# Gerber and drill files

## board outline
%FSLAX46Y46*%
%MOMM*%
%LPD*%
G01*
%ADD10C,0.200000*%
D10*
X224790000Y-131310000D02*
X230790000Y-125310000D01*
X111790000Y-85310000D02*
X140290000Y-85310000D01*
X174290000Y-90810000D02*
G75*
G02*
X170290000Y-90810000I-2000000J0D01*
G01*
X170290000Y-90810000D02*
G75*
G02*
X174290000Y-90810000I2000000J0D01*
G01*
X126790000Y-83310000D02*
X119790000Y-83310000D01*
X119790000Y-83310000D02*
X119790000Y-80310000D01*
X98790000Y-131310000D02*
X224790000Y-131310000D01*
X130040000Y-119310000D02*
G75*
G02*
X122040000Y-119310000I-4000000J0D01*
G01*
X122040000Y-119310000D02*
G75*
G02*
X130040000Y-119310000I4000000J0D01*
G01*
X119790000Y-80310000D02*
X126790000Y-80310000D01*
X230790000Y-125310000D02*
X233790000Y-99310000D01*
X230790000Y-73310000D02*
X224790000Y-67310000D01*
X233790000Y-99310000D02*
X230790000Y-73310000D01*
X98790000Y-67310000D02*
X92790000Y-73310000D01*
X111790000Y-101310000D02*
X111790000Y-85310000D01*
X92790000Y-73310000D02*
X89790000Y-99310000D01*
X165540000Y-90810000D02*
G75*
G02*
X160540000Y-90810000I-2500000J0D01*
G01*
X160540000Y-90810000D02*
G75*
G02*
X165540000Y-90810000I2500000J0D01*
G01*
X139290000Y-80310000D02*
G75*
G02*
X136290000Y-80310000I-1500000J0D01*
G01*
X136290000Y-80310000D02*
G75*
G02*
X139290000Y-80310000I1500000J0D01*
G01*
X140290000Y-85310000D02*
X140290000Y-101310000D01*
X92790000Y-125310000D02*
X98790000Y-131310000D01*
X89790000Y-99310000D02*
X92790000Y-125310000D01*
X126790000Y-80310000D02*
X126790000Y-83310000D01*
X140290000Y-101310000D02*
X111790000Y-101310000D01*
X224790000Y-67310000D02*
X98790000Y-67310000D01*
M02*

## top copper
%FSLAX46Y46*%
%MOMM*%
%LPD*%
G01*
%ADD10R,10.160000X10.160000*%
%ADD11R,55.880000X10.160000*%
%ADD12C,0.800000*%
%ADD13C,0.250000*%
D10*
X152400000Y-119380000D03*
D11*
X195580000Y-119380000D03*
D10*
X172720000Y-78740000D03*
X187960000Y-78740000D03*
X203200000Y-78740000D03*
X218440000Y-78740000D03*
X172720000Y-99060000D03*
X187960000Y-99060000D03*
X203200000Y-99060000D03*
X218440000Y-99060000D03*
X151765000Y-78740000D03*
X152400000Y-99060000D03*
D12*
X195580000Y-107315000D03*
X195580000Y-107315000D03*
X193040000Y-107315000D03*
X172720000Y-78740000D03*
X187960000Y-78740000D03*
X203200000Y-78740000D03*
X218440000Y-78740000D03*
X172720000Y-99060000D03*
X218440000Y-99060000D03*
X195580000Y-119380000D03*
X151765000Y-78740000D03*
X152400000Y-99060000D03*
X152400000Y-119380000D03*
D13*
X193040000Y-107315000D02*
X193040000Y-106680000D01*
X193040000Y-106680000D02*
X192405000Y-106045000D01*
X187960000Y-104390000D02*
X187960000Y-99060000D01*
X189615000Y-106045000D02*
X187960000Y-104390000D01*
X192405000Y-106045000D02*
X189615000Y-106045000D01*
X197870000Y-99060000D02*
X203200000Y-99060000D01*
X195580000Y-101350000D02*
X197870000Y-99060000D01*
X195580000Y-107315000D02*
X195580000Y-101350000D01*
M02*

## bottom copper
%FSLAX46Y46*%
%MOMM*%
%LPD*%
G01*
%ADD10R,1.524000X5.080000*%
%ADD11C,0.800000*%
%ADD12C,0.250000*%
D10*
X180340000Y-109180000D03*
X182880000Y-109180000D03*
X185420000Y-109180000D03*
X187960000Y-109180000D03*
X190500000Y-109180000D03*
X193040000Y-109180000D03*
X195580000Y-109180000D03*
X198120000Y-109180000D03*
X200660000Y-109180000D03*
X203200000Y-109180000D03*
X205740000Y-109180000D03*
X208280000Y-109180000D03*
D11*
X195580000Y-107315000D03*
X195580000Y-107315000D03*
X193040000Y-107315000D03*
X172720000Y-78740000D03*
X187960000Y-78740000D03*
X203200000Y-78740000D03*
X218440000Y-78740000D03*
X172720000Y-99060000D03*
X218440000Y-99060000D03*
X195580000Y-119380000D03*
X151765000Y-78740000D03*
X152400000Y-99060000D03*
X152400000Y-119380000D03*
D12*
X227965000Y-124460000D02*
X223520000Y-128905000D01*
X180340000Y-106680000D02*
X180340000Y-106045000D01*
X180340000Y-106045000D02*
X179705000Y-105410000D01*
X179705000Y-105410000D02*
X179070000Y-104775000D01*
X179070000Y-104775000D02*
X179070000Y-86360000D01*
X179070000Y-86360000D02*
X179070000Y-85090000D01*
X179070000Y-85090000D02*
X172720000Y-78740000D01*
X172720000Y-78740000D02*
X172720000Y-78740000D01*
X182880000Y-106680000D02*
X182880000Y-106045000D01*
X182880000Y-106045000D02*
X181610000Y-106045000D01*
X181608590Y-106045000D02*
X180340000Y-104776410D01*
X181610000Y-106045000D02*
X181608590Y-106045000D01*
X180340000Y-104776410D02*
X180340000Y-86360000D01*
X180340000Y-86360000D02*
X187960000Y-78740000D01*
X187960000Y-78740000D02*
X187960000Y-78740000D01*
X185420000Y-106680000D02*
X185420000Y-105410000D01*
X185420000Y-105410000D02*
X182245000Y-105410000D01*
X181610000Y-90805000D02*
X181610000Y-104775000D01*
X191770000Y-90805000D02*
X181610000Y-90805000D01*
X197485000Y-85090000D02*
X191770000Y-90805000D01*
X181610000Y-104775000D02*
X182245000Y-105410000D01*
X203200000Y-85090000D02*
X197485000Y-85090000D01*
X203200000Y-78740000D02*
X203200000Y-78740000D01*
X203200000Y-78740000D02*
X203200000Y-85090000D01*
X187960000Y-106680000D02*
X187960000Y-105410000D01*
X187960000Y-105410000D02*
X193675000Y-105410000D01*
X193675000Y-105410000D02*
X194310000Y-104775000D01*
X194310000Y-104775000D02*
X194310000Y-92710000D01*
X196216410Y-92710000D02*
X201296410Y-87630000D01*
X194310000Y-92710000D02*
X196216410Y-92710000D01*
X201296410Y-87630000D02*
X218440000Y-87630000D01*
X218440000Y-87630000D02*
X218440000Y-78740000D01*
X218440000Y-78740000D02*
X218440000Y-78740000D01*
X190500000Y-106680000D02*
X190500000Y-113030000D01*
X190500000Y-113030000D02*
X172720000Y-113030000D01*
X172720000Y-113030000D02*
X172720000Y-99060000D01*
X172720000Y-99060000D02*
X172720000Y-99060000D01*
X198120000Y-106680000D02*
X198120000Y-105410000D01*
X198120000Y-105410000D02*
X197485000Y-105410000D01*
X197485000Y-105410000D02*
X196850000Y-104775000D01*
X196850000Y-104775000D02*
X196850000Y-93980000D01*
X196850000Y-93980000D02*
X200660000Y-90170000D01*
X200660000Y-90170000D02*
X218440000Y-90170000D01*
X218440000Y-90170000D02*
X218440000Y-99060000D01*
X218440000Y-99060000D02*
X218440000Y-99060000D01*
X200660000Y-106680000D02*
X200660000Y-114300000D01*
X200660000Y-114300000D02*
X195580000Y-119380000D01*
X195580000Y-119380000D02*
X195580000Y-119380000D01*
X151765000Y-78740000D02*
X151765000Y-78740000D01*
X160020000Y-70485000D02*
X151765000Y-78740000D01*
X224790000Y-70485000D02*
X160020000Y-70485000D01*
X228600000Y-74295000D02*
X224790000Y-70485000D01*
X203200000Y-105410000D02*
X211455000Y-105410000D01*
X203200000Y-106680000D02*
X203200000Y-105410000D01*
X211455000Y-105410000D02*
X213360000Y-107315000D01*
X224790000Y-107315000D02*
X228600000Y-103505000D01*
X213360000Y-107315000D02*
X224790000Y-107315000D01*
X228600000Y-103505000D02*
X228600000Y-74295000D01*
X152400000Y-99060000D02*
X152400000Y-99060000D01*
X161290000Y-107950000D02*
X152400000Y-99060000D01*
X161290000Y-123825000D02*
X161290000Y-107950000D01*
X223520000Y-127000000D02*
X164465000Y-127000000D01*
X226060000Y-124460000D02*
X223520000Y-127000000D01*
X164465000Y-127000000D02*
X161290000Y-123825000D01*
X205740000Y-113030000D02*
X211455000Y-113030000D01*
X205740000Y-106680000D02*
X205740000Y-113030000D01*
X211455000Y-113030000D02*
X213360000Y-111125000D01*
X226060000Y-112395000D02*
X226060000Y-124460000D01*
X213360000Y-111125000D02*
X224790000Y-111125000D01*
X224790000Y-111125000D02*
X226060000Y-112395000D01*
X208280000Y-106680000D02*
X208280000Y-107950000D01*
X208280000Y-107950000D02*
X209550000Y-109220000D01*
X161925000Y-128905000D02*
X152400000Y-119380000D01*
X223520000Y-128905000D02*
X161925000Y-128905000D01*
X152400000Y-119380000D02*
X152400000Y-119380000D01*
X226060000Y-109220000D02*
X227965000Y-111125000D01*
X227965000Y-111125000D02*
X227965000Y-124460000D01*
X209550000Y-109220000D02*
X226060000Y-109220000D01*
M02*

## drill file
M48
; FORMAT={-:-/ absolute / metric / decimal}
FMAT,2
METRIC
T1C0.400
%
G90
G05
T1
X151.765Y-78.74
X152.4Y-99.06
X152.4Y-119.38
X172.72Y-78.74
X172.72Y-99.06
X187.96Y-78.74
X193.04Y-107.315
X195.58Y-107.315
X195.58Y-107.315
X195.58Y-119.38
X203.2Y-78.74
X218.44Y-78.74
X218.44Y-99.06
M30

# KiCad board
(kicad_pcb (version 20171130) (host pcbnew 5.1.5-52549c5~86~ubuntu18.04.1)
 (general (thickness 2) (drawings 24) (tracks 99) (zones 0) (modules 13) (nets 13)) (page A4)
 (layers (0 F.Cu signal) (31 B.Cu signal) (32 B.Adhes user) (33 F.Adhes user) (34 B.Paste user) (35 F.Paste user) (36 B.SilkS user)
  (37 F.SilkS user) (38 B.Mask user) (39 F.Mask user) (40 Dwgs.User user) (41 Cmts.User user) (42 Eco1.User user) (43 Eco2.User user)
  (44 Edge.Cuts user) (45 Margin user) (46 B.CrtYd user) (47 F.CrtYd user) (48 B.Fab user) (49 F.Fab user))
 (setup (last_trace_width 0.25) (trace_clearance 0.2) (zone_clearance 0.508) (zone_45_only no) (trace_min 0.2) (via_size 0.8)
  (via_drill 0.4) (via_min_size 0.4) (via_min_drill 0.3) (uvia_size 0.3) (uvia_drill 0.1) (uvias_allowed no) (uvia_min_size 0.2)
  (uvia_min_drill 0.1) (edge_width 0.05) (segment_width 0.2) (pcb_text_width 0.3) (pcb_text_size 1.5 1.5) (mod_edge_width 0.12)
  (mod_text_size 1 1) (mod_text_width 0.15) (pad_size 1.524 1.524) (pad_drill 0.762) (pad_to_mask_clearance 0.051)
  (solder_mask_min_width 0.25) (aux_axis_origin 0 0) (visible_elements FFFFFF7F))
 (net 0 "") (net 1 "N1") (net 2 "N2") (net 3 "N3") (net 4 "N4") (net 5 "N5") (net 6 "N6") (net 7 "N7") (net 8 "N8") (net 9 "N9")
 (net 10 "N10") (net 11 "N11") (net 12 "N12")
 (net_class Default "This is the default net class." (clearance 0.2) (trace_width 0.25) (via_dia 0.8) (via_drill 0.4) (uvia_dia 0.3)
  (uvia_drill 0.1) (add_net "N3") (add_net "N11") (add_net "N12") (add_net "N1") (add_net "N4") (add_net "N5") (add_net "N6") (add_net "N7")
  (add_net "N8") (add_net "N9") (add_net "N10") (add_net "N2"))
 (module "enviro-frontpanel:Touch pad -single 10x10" (layer F.Cu) (at 152.4 127)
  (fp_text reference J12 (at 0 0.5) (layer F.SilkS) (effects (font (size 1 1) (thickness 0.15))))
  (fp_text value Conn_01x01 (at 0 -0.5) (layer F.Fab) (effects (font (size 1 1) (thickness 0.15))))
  (pad 1 smd rect (at 0 -7.62) (size 10.16 10.16) (layers F.Cu F.Paste F.Mask) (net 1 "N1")))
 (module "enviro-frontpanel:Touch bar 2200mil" (layer F.Cu) (at 195.58 127)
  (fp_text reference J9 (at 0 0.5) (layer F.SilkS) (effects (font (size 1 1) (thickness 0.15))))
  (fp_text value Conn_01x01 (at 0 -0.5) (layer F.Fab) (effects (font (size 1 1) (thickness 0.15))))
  (pad 1 smd rect (at 0 -7.62) (size 55.88 10.16) (layers F.Cu F.Paste F.Mask) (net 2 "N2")))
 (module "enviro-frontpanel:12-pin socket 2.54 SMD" (layer B.Cu) (at 210.82 106.68 270)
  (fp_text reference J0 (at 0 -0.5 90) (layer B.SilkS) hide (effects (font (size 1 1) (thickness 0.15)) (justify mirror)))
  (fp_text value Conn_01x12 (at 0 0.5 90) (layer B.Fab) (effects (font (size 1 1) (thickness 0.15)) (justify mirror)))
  (pad 1 smd rect (at 0 30.48 270) (size 5.08 1.524) (drill (offset 2.5 0)) (layers B.Cu B.Paste B.Mask) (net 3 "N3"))
  (pad 2 smd rect (at 0 27.94 270) (size 5.08 1.524) (drill (offset 2.5 0)) (layers B.Cu B.Paste B.Mask) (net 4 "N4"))
  (pad 3 smd rect (at 0 25.4 270) (size 5.08 1.524) (drill (offset 2.5 0)) (layers B.Cu B.Paste B.Mask) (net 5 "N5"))
  (pad 4 smd rect (at 0 22.86 270) (size 5.08 1.524) (drill (offset 2.5 0)) (layers B.Cu B.Paste B.Mask) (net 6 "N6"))
  (pad 5 smd rect (at 0 20.32 270) (size 5.08 1.524) (drill (offset 2.5 0)) (layers B.Cu B.Paste B.Mask) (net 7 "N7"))
  (pad 6 smd rect (at 0 17.78 270) (size 5.08 1.524) (drill (offset 2.5 0)) (layers B.Cu B.Paste B.Mask) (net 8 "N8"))
  (pad 7 smd rect (at 0 15.24 270) (size 5.08 1.524) (drill (offset 2.5 0)) (layers B.Cu B.Paste B.Mask) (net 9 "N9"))
  (pad 8 smd rect (at 0 12.7 270) (size 5.08 1.524) (drill (offset 2.5 0)) (layers B.Cu B.Paste B.Mask) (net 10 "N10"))
  (pad 9 smd rect (at 0 10.16 270) (size 5.08 1.524) (drill (offset 2.5 0)) (layers B.Cu B.Paste B.Mask) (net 2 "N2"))
  (pad 10 smd rect (at 0 7.62 270) (size 5.08 1.524) (drill (offset 2.5 0)) (layers B.Cu B.Paste B.Mask) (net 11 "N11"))
  (pad 11 smd rect (at 0 5.08 270) (size 5.08 1.524) (drill (offset 2.5 0)) (layers B.Cu B.Paste B.Mask) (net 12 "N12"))
  (pad 12 smd rect (at 0 2.54 270) (size 5.08 1.524) (drill (offset 2.5 0)) (layers B.Cu B.Paste B.Mask) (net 1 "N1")))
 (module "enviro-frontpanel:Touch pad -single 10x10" (layer F.Cu) (at 172.72 86.36)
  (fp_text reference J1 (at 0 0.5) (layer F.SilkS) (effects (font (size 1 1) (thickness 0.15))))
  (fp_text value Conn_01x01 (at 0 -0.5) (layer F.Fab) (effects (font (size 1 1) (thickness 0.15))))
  (pad 1 smd rect (at 0 -7.62) (size 10.16 10.16) (layers F.Cu F.Paste F.Mask) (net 3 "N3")))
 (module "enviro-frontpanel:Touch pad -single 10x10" (layer F.Cu) (at 187.96 86.36)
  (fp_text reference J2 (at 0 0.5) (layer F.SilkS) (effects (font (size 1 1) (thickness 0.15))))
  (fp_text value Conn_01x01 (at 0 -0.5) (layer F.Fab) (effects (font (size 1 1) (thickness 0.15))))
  (pad 1 smd rect (at 0 -7.62) (size 10.16 10.16) (layers F.Cu F.Paste F.Mask) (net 4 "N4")))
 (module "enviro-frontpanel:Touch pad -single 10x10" (layer F.Cu) (at 203.2 86.36)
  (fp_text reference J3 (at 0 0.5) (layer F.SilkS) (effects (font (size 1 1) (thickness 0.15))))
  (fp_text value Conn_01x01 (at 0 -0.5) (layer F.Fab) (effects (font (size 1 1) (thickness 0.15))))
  (pad 1 smd rect (at 0 -7.62) (size 10.16 10.16) (layers F.Cu F.Paste F.Mask) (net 5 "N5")))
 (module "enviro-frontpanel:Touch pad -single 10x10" (layer F.Cu) (at 218.44 86.36)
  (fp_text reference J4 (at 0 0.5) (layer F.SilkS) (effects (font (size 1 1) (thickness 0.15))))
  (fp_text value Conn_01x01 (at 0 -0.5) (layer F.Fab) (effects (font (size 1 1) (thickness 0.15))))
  (pad 1 smd rect (at 0 -7.62) (size 10.16 10.16) (layers F.Cu F.Paste F.Mask) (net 6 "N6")))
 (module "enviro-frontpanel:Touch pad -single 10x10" (layer F.Cu) (at 172.72 106.68)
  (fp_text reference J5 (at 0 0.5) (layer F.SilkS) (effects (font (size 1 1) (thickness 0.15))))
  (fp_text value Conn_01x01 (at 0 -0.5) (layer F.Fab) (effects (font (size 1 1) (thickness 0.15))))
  (pad 1 smd rect (at 0 -7.62) (size 10.16 10.16) (layers F.Cu F.Paste F.Mask) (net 7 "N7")))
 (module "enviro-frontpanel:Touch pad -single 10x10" (layer F.Cu) (at 187.96 106.68)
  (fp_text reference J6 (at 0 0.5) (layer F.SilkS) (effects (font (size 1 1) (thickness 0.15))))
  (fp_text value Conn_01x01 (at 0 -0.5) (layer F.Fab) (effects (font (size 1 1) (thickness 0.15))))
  (pad 1 smd rect (at 0 -7.62) (size 10.16 10.16) (layers F.Cu F.Paste F.Mask) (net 8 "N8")))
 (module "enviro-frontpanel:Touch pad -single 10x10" (layer F.Cu) (at 203.2 106.68)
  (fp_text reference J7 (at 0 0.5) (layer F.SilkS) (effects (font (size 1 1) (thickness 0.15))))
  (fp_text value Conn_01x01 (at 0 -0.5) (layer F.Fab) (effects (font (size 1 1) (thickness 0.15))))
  (pad 1 smd rect (at 0 -7.62) (size 10.16 10.16) (layers F.Cu F.Paste F.Mask) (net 9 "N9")))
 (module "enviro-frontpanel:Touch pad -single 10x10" (layer F.Cu) (at 218.44 106.68)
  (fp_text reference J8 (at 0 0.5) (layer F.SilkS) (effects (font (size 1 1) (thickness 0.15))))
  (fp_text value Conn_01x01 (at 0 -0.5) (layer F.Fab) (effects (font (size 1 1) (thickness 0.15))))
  (pad 1 smd rect (at 0 -7.62) (size 10.16 10.16) (layers F.Cu F.Paste F.Mask) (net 10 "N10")))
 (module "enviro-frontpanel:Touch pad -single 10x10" (layer F.Cu) (at 151.765 86.36)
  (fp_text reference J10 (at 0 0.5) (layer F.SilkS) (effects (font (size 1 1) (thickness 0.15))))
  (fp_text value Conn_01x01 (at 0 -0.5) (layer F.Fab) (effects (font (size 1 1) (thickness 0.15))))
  (pad 1 smd rect (at 0 -7.62) (size 10.16 10.16) (layers F.Cu F.Paste F.Mask) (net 11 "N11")))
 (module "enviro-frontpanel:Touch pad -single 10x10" (layer F.Cu) (at 152.4 106.68)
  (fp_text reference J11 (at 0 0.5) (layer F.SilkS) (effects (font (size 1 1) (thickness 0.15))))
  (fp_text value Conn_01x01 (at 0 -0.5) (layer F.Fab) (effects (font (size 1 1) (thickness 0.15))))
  (pad 1 smd rect (at 0 -7.62) (size 10.16 10.16) (layers F.Cu F.Paste F.Mask) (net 12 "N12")))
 (gr_line (start 224.79 131.31) (end 230.79 125.31) (layer Edge.Cuts) (width 0.2))
 (gr_line (start 111.79 85.31) (end 140.29 85.31) (layer Edge.Cuts) (width 0.2))
 (gr_circle (center 172.29 90.81) (end 174.29 90.81) (layer Edge.Cuts) (width 0.2))
 (gr_line (start 126.79 83.31) (end 119.79 83.31) (layer Edge.Cuts) (width 0.2))
 (gr_line (start 119.79 83.31) (end 119.79 80.31) (layer Edge.Cuts) (width 0.2))
 (gr_line (start 98.79 131.31) (end 224.79 131.31) (layer Edge.Cuts) (width 0.2))
 (gr_circle (center 126.04 119.31) (end 130.04 119.31) (layer Edge.Cuts) (width 0.2))
 (gr_line (start 119.79 80.31) (end 126.79 80.31) (layer Edge.Cuts) (width 0.2))
 (gr_line (start 230.79 125.31) (end 233.79 99.31) (layer Edge.Cuts) (width 0.2))
 (gr_line (start 230.79 73.31) (end 224.79 67.31) (layer Edge.Cuts) (width 0.2))
 (gr_line (start 233.79 99.31) (end 230.79 73.31) (layer Edge.Cuts) (width 0.2))
 (gr_line (start 98.79 67.31) (end 92.79 73.31) (layer Edge.Cuts) (width 0.2))
 (gr_line (start 111.79 101.31) (end 111.79 85.31) (layer Edge.Cuts) (width 0.2))
 (gr_line (start 92.79 73.31) (end 89.79 99.31) (layer Edge.Cuts) (width 0.2))
 (gr_circle (center 163.04 90.81) (end 165.54 90.81) (layer Edge.Cuts) (width 0.2))
 (gr_circle (center 137.79 80.31) (end 139.29 80.31) (layer Edge.Cuts) (width 0.2))
 (gr_line (start 140.29 85.31) (end 140.29 101.31) (layer Edge.Cuts) (width 0.2))
 (gr_line (start 92.79 125.31) (end 98.79 131.31) (layer Edge.Cuts) (width 0.2))
 (gr_line (start 89.79 99.31) (end 92.79 125.31) (layer Edge.Cuts) (width 0.2))
 (gr_line (start 126.79 80.31) (end 126.79 83.31) (layer Edge.Cuts) (width 0.2))
 (gr_line (start 140.29 101.31) (end 111.79 101.31) (layer Edge.Cuts) (width 0.2))
 (gr_line (start 224.79 67.31) (end 98.79 67.31) (layer Edge.Cuts) (width 0.2))
 (segment (start 227.965 124.46) (end 223.52 128.905) (width 0.25) (layer B.Cu) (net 1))
 (via (at 195.58 107.315) (size 0.8) (drill 0.4) (layers F.Cu B.Cu) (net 9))
 (via (at 195.58 107.315) (size 0.8) (drill 0.4) (layers F.Cu B.Cu) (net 9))
 (via (at 193.04 107.315) (size 0.8) (drill 0.4) (layers F.Cu B.Cu) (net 8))
 (segment (start 180.34 106.68) (end 180.34 106.045) (width 0.25) (layer B.Cu) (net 3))
 (segment (start 180.34 106.045) (end 179.705 105.41) (width 0.25) (layer B.Cu) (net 3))
 (segment (start 179.705 105.41) (end 179.07 104.775) (width 0.25) (layer B.Cu) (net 3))
 (segment (start 179.07 104.775) (end 179.07 86.36) (width 0.25) (layer B.Cu) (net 3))
 (segment (start 179.07 86.36) (end 179.07 85.09) (width 0.25) (layer B.Cu) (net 3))
 (segment (start 179.07 85.09) (end 172.72 78.74) (width 0.25) (layer B.Cu) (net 3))
 (segment (start 172.72 78.74) (end 172.72 78.74) (width 0.25) (layer B.Cu) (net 3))
 (via (at 172.72 78.74) (size 0.8) (drill 0.4) (layers F.Cu B.Cu) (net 3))
 (segment (start 182.88 106.68) (end 182.88 106.045) (width 0.25) (layer B.Cu) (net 4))
 (segment (start 182.88 106.045) (end 181.61 106.045) (width 0.25) (layer B.Cu) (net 4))
 (segment (start 181.60859 106.045) (end 180.34 104.77641) (width 0.25) (layer B.Cu) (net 4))
 (segment (start 181.61 106.045) (end 181.60859 106.045) (width 0.25) (layer B.Cu) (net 4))
 (segment (start 180.34 104.77641) (end 180.34 86.36) (width 0.25) (layer B.Cu) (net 4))
 (segment (start 180.34 86.36) (end 187.96 78.74) (width 0.25) (layer B.Cu) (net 4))
 (segment (start 187.96 78.74) (end 187.96 78.74) (width 0.25) (layer B.Cu) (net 4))
 (via (at 187.96 78.74) (size 0.8) (drill 0.4) (layers F.Cu B.Cu) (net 4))
 (segment (start 185.42 106.68) (end 185.42 105.41) (width 0.25) (layer B.Cu) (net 5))
 (segment (start 185.42 105.41) (end 182.245 105.41) (width 0.25) (layer B.Cu) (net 5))
 (segment (start 181.61 90.805) (end 181.61 104.775) (width 0.25) (layer B.Cu) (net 5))
 (segment (start 191.77 90.805) (end 181.61 90.805) (width 0.25) (layer B.Cu) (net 5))
 (segment (start 197.485 85.09) (end 191.77 90.805) (width 0.25) (layer B.Cu) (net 5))
 (segment (start 181.61 104.775) (end 182.245 105.41) (width 0.25) (layer B.Cu) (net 5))
 (segment (start 203.2 85.09) (end 197.485 85.09) (width 0.25) (layer B.Cu) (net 5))
 (segment (start 203.2 78.74) (end 203.2 78.74) (width 0.25) (layer B.Cu) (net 5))
 (segment (start 203.2 78.74) (end 203.2 85.09) (width 0.25) (layer B.Cu) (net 5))
 (via (at 203.2 78.74) (size 0.8) (drill 0.4) (layers F.Cu B.Cu) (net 5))
 (segment (start 187.96 106.68) (end 187.96 105.41) (width 0.25) (layer B.Cu) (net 6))
 (segment (start 187.96 105.41) (end 193.675 105.41) (width 0.25) (layer B.Cu) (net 6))
 (segment (start 193.675 105.41) (end 194.31 104.775) (width 0.25) (layer B.Cu) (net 6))
 (segment (start 194.31 104.775) (end 194.31 92.71) (width 0.25) (layer B.Cu) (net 6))
 (segment (start 196.21641 92.71) (end 201.29641 87.63) (width 0.25) (layer B.Cu) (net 6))
 (segment (start 194.31 92.71) (end 196.21641 92.71) (width 0.25) (layer B.Cu) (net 6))
 (segment (start 201.29641 87.63) (end 218.44 87.63) (width 0.25) (layer B.Cu) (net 6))
 (segment (start 218.44 87.63) (end 218.44 78.74) (width 0.25) (layer B.Cu) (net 6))
 (segment (start 218.44 78.74) (end 218.44 78.74) (width 0.25) (layer B.Cu) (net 6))
 (via (at 218.44 78.74) (size 0.8) (drill 0.4) (layers F.Cu B.Cu) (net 6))
 (segment (start 190.5 106.68) (end 190.5 113.03) (width 0.25) (layer B.Cu) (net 7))
 (segment (start 190.5 113.03) (end 172.72 113.03) (width 0.25) (layer B.Cu) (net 7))
 (segment (start 172.72 113.03) (end 172.72 99.06) (width 0.25) (layer B.Cu) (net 7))
 (segment (start 172.72 99.06) (end 172.72 99.06) (width 0.25) (layer B.Cu) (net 7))
 (via (at 172.72 99.06) (size 0.8) (drill 0.4) (layers F.Cu B.Cu) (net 7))
 (segment (start 193.04 107.315) (end 193.04 106.68) (width 0.25) (layer F.Cu) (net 8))
 (segment (start 193.04 106.68) (end 192.405 106.045) (width 0.25) (layer F.Cu) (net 8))
 (segment (start 187.96 104.39) (end 187.96 99.06) (width 0.25) (layer F.Cu) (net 8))
 (segment (start 189.615 106.045) (end 187.96 104.39) (width 0.25) (layer F.Cu) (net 8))
 (segment (start 192.405 106.045) (end 189.615 106.045) (width 0.25) (layer F.Cu) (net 8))
 (segment (start 197.87 99.06) (end 203.2 99.06) (width 0.25) (layer F.Cu) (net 9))
 (segment (start 195.58 101.35) (end 197.87 99.06) (width 0.25) (layer F.Cu) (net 9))
 (segment (start 195.58 107.315) (end 195.58 101.35) (width 0.25) (layer F.Cu) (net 9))
 (segment (start 198.12 106.68) (end 198.12 105.41) (width 0.25) (layer B.Cu) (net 10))
 (segment (start 198.12 105.41) (end 197.485 105.41) (width 0.25) (layer B.Cu) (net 10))
 (segment (start 197.485 105.41) (end 196.85 104.775) (width 0.25) (layer B.Cu) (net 10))
 (segment (start 196.85 104.775) (end 196.85 93.98) (width 0.25) (layer B.Cu) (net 10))
 (segment (start 196.85 93.98) (end 200.66 90.17) (width 0.25) (layer B.Cu) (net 10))
 (segment (start 200.66 90.17) (end 218.44 90.17) (width 0.25) (layer B.Cu) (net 10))
 (segment (start 218.44 90.17) (end 218.44 99.06) (width 0.25) (layer B.Cu) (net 10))
 (segment (start 218.44 99.06) (end 218.44 99.06) (width 0.25) (layer B.Cu) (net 10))
 (via (at 218.44 99.06) (size 0.8) (drill 0.4) (layers F.Cu B.Cu) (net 10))
 (segment (start 200.66 106.68) (end 200.66 114.3) (width 0.25) (layer B.Cu) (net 2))
 (segment (start 200.66 114.3) (end 195.58 119.38) (width 0.25) (layer B.Cu) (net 2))
 (segment (start 195.58 119.38) (end 195.58 119.38) (width 0.25) (layer B.Cu) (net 2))
 (via (at 195.58 119.38) (size 0.8) (drill 0.4) (layers F.Cu B.Cu) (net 2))
 (segment (start 151.765 78.74) (end 151.765 78.74) (width 0.25) (layer B.Cu) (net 11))
 (via (at 151.765 78.74) (size 0.8) (drill 0.4) (layers F.Cu B.Cu) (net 11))
 (segment (start 160.02 70.485) (end 151.765 78.74) (width 0.25) (layer B.Cu) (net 11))
 (segment (start 224.79 70.485) (end 160.02 70.485) (width 0.25) (layer B.Cu) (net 11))
 (segment (start 228.6 74.295) (end 224.79 70.485) (width 0.25) (layer B.Cu) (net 11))
 (segment (start 203.2 105.41) (end 211.455 105.41) (width 0.25) (layer B.Cu) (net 11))
 (segment (start 203.2 106.68) (end 203.2 105.41) (width 0.25) (layer B.Cu) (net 11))
 (segment (start 211.455 105.41) (end 213.36 107.315) (width 0.25) (layer B.Cu) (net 11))
 (segment (start 224.79 107.315) (end 228.6 103.505) (width 0.25) (layer B.Cu) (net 11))
 (segment (start 213.36 107.315) (end 224.79 107.315) (width 0.25) (layer B.Cu) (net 11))
 (segment (start 228.6 103.505) (end 228.6 74.295) (width 0.25) (layer B.Cu) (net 11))
 (segment (start 152.4 99.06) (end 152.4 99.06) (width 0.25) (layer B.Cu) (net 12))
 (via (at 152.4 99.06) (size 0.8) (drill 0.4) (layers F.Cu B.Cu) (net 12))
 (segment (start 161.29 107.95) (end 152.4 99.06) (width 0.25) (layer B.Cu) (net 12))
 (segment (start 161.29 123.825) (end 161.29 107.95) (width 0.25) (layer B.Cu) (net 12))
 (segment (start 223.52 127) (end 164.465 127) (width 0.25) (layer B.Cu) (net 12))
 (segment (start 226.06 124.46) (end 223.52 127) (width 0.25) (layer B.Cu) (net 12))
 (segment (start 164.465 127) (end 161.29 123.825) (width 0.25) (layer B.Cu) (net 12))
 (segment (start 205.74 113.03) (end 211.455 113.03) (width 0.25) (layer B.Cu) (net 12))
 (segment (start 205.74 106.68) (end 205.74 113.03) (width 0.25) (layer B.Cu) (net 12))
 (segment (start 211.455 113.03) (end 213.36 111.125) (width 0.25) (layer B.Cu) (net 12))
 (segment (start 226.06 112.395) (end 226.06 124.46) (width 0.25) (layer B.Cu) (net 12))
 (segment (start 213.36 111.125) (end 224.79 111.125) (width 0.25) (layer B.Cu) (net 12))
 (segment (start 224.79 111.125) (end 226.06 112.395) (width 0.25) (layer B.Cu) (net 12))
 (segment (start 208.28 106.68) (end 208.28 107.95) (width 0.25) (layer B.Cu) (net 1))
 (segment (start 208.28 107.95) (end 209.55 109.22) (width 0.25) (layer B.Cu) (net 1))
 (segment (start 161.925 128.905) (end 152.4 119.38) (width 0.25) (layer B.Cu) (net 1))
 (segment (start 223.52 128.905) (end 161.925 128.905) (width 0.25) (layer B.Cu) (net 1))
 (segment (start 152.4 119.38) (end 152.4 119.38) (width 0.25) (layer B.Cu) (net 1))
 (via (at 152.4 119.38) (size 0.8) (drill 0.4) (layers F.Cu B.Cu) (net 1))
 (segment (start 226.06 109.22) (end 227.965 111.125) (width 0.25) (layer B.Cu) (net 1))
 (segment (start 227.965 111.125) (end 227.965 124.46) (width 0.25) (layer B.Cu) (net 1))
 (segment (start 209.55 109.22) (end 226.06 109.22) (width 0.25) (layer B.Cu) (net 1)))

